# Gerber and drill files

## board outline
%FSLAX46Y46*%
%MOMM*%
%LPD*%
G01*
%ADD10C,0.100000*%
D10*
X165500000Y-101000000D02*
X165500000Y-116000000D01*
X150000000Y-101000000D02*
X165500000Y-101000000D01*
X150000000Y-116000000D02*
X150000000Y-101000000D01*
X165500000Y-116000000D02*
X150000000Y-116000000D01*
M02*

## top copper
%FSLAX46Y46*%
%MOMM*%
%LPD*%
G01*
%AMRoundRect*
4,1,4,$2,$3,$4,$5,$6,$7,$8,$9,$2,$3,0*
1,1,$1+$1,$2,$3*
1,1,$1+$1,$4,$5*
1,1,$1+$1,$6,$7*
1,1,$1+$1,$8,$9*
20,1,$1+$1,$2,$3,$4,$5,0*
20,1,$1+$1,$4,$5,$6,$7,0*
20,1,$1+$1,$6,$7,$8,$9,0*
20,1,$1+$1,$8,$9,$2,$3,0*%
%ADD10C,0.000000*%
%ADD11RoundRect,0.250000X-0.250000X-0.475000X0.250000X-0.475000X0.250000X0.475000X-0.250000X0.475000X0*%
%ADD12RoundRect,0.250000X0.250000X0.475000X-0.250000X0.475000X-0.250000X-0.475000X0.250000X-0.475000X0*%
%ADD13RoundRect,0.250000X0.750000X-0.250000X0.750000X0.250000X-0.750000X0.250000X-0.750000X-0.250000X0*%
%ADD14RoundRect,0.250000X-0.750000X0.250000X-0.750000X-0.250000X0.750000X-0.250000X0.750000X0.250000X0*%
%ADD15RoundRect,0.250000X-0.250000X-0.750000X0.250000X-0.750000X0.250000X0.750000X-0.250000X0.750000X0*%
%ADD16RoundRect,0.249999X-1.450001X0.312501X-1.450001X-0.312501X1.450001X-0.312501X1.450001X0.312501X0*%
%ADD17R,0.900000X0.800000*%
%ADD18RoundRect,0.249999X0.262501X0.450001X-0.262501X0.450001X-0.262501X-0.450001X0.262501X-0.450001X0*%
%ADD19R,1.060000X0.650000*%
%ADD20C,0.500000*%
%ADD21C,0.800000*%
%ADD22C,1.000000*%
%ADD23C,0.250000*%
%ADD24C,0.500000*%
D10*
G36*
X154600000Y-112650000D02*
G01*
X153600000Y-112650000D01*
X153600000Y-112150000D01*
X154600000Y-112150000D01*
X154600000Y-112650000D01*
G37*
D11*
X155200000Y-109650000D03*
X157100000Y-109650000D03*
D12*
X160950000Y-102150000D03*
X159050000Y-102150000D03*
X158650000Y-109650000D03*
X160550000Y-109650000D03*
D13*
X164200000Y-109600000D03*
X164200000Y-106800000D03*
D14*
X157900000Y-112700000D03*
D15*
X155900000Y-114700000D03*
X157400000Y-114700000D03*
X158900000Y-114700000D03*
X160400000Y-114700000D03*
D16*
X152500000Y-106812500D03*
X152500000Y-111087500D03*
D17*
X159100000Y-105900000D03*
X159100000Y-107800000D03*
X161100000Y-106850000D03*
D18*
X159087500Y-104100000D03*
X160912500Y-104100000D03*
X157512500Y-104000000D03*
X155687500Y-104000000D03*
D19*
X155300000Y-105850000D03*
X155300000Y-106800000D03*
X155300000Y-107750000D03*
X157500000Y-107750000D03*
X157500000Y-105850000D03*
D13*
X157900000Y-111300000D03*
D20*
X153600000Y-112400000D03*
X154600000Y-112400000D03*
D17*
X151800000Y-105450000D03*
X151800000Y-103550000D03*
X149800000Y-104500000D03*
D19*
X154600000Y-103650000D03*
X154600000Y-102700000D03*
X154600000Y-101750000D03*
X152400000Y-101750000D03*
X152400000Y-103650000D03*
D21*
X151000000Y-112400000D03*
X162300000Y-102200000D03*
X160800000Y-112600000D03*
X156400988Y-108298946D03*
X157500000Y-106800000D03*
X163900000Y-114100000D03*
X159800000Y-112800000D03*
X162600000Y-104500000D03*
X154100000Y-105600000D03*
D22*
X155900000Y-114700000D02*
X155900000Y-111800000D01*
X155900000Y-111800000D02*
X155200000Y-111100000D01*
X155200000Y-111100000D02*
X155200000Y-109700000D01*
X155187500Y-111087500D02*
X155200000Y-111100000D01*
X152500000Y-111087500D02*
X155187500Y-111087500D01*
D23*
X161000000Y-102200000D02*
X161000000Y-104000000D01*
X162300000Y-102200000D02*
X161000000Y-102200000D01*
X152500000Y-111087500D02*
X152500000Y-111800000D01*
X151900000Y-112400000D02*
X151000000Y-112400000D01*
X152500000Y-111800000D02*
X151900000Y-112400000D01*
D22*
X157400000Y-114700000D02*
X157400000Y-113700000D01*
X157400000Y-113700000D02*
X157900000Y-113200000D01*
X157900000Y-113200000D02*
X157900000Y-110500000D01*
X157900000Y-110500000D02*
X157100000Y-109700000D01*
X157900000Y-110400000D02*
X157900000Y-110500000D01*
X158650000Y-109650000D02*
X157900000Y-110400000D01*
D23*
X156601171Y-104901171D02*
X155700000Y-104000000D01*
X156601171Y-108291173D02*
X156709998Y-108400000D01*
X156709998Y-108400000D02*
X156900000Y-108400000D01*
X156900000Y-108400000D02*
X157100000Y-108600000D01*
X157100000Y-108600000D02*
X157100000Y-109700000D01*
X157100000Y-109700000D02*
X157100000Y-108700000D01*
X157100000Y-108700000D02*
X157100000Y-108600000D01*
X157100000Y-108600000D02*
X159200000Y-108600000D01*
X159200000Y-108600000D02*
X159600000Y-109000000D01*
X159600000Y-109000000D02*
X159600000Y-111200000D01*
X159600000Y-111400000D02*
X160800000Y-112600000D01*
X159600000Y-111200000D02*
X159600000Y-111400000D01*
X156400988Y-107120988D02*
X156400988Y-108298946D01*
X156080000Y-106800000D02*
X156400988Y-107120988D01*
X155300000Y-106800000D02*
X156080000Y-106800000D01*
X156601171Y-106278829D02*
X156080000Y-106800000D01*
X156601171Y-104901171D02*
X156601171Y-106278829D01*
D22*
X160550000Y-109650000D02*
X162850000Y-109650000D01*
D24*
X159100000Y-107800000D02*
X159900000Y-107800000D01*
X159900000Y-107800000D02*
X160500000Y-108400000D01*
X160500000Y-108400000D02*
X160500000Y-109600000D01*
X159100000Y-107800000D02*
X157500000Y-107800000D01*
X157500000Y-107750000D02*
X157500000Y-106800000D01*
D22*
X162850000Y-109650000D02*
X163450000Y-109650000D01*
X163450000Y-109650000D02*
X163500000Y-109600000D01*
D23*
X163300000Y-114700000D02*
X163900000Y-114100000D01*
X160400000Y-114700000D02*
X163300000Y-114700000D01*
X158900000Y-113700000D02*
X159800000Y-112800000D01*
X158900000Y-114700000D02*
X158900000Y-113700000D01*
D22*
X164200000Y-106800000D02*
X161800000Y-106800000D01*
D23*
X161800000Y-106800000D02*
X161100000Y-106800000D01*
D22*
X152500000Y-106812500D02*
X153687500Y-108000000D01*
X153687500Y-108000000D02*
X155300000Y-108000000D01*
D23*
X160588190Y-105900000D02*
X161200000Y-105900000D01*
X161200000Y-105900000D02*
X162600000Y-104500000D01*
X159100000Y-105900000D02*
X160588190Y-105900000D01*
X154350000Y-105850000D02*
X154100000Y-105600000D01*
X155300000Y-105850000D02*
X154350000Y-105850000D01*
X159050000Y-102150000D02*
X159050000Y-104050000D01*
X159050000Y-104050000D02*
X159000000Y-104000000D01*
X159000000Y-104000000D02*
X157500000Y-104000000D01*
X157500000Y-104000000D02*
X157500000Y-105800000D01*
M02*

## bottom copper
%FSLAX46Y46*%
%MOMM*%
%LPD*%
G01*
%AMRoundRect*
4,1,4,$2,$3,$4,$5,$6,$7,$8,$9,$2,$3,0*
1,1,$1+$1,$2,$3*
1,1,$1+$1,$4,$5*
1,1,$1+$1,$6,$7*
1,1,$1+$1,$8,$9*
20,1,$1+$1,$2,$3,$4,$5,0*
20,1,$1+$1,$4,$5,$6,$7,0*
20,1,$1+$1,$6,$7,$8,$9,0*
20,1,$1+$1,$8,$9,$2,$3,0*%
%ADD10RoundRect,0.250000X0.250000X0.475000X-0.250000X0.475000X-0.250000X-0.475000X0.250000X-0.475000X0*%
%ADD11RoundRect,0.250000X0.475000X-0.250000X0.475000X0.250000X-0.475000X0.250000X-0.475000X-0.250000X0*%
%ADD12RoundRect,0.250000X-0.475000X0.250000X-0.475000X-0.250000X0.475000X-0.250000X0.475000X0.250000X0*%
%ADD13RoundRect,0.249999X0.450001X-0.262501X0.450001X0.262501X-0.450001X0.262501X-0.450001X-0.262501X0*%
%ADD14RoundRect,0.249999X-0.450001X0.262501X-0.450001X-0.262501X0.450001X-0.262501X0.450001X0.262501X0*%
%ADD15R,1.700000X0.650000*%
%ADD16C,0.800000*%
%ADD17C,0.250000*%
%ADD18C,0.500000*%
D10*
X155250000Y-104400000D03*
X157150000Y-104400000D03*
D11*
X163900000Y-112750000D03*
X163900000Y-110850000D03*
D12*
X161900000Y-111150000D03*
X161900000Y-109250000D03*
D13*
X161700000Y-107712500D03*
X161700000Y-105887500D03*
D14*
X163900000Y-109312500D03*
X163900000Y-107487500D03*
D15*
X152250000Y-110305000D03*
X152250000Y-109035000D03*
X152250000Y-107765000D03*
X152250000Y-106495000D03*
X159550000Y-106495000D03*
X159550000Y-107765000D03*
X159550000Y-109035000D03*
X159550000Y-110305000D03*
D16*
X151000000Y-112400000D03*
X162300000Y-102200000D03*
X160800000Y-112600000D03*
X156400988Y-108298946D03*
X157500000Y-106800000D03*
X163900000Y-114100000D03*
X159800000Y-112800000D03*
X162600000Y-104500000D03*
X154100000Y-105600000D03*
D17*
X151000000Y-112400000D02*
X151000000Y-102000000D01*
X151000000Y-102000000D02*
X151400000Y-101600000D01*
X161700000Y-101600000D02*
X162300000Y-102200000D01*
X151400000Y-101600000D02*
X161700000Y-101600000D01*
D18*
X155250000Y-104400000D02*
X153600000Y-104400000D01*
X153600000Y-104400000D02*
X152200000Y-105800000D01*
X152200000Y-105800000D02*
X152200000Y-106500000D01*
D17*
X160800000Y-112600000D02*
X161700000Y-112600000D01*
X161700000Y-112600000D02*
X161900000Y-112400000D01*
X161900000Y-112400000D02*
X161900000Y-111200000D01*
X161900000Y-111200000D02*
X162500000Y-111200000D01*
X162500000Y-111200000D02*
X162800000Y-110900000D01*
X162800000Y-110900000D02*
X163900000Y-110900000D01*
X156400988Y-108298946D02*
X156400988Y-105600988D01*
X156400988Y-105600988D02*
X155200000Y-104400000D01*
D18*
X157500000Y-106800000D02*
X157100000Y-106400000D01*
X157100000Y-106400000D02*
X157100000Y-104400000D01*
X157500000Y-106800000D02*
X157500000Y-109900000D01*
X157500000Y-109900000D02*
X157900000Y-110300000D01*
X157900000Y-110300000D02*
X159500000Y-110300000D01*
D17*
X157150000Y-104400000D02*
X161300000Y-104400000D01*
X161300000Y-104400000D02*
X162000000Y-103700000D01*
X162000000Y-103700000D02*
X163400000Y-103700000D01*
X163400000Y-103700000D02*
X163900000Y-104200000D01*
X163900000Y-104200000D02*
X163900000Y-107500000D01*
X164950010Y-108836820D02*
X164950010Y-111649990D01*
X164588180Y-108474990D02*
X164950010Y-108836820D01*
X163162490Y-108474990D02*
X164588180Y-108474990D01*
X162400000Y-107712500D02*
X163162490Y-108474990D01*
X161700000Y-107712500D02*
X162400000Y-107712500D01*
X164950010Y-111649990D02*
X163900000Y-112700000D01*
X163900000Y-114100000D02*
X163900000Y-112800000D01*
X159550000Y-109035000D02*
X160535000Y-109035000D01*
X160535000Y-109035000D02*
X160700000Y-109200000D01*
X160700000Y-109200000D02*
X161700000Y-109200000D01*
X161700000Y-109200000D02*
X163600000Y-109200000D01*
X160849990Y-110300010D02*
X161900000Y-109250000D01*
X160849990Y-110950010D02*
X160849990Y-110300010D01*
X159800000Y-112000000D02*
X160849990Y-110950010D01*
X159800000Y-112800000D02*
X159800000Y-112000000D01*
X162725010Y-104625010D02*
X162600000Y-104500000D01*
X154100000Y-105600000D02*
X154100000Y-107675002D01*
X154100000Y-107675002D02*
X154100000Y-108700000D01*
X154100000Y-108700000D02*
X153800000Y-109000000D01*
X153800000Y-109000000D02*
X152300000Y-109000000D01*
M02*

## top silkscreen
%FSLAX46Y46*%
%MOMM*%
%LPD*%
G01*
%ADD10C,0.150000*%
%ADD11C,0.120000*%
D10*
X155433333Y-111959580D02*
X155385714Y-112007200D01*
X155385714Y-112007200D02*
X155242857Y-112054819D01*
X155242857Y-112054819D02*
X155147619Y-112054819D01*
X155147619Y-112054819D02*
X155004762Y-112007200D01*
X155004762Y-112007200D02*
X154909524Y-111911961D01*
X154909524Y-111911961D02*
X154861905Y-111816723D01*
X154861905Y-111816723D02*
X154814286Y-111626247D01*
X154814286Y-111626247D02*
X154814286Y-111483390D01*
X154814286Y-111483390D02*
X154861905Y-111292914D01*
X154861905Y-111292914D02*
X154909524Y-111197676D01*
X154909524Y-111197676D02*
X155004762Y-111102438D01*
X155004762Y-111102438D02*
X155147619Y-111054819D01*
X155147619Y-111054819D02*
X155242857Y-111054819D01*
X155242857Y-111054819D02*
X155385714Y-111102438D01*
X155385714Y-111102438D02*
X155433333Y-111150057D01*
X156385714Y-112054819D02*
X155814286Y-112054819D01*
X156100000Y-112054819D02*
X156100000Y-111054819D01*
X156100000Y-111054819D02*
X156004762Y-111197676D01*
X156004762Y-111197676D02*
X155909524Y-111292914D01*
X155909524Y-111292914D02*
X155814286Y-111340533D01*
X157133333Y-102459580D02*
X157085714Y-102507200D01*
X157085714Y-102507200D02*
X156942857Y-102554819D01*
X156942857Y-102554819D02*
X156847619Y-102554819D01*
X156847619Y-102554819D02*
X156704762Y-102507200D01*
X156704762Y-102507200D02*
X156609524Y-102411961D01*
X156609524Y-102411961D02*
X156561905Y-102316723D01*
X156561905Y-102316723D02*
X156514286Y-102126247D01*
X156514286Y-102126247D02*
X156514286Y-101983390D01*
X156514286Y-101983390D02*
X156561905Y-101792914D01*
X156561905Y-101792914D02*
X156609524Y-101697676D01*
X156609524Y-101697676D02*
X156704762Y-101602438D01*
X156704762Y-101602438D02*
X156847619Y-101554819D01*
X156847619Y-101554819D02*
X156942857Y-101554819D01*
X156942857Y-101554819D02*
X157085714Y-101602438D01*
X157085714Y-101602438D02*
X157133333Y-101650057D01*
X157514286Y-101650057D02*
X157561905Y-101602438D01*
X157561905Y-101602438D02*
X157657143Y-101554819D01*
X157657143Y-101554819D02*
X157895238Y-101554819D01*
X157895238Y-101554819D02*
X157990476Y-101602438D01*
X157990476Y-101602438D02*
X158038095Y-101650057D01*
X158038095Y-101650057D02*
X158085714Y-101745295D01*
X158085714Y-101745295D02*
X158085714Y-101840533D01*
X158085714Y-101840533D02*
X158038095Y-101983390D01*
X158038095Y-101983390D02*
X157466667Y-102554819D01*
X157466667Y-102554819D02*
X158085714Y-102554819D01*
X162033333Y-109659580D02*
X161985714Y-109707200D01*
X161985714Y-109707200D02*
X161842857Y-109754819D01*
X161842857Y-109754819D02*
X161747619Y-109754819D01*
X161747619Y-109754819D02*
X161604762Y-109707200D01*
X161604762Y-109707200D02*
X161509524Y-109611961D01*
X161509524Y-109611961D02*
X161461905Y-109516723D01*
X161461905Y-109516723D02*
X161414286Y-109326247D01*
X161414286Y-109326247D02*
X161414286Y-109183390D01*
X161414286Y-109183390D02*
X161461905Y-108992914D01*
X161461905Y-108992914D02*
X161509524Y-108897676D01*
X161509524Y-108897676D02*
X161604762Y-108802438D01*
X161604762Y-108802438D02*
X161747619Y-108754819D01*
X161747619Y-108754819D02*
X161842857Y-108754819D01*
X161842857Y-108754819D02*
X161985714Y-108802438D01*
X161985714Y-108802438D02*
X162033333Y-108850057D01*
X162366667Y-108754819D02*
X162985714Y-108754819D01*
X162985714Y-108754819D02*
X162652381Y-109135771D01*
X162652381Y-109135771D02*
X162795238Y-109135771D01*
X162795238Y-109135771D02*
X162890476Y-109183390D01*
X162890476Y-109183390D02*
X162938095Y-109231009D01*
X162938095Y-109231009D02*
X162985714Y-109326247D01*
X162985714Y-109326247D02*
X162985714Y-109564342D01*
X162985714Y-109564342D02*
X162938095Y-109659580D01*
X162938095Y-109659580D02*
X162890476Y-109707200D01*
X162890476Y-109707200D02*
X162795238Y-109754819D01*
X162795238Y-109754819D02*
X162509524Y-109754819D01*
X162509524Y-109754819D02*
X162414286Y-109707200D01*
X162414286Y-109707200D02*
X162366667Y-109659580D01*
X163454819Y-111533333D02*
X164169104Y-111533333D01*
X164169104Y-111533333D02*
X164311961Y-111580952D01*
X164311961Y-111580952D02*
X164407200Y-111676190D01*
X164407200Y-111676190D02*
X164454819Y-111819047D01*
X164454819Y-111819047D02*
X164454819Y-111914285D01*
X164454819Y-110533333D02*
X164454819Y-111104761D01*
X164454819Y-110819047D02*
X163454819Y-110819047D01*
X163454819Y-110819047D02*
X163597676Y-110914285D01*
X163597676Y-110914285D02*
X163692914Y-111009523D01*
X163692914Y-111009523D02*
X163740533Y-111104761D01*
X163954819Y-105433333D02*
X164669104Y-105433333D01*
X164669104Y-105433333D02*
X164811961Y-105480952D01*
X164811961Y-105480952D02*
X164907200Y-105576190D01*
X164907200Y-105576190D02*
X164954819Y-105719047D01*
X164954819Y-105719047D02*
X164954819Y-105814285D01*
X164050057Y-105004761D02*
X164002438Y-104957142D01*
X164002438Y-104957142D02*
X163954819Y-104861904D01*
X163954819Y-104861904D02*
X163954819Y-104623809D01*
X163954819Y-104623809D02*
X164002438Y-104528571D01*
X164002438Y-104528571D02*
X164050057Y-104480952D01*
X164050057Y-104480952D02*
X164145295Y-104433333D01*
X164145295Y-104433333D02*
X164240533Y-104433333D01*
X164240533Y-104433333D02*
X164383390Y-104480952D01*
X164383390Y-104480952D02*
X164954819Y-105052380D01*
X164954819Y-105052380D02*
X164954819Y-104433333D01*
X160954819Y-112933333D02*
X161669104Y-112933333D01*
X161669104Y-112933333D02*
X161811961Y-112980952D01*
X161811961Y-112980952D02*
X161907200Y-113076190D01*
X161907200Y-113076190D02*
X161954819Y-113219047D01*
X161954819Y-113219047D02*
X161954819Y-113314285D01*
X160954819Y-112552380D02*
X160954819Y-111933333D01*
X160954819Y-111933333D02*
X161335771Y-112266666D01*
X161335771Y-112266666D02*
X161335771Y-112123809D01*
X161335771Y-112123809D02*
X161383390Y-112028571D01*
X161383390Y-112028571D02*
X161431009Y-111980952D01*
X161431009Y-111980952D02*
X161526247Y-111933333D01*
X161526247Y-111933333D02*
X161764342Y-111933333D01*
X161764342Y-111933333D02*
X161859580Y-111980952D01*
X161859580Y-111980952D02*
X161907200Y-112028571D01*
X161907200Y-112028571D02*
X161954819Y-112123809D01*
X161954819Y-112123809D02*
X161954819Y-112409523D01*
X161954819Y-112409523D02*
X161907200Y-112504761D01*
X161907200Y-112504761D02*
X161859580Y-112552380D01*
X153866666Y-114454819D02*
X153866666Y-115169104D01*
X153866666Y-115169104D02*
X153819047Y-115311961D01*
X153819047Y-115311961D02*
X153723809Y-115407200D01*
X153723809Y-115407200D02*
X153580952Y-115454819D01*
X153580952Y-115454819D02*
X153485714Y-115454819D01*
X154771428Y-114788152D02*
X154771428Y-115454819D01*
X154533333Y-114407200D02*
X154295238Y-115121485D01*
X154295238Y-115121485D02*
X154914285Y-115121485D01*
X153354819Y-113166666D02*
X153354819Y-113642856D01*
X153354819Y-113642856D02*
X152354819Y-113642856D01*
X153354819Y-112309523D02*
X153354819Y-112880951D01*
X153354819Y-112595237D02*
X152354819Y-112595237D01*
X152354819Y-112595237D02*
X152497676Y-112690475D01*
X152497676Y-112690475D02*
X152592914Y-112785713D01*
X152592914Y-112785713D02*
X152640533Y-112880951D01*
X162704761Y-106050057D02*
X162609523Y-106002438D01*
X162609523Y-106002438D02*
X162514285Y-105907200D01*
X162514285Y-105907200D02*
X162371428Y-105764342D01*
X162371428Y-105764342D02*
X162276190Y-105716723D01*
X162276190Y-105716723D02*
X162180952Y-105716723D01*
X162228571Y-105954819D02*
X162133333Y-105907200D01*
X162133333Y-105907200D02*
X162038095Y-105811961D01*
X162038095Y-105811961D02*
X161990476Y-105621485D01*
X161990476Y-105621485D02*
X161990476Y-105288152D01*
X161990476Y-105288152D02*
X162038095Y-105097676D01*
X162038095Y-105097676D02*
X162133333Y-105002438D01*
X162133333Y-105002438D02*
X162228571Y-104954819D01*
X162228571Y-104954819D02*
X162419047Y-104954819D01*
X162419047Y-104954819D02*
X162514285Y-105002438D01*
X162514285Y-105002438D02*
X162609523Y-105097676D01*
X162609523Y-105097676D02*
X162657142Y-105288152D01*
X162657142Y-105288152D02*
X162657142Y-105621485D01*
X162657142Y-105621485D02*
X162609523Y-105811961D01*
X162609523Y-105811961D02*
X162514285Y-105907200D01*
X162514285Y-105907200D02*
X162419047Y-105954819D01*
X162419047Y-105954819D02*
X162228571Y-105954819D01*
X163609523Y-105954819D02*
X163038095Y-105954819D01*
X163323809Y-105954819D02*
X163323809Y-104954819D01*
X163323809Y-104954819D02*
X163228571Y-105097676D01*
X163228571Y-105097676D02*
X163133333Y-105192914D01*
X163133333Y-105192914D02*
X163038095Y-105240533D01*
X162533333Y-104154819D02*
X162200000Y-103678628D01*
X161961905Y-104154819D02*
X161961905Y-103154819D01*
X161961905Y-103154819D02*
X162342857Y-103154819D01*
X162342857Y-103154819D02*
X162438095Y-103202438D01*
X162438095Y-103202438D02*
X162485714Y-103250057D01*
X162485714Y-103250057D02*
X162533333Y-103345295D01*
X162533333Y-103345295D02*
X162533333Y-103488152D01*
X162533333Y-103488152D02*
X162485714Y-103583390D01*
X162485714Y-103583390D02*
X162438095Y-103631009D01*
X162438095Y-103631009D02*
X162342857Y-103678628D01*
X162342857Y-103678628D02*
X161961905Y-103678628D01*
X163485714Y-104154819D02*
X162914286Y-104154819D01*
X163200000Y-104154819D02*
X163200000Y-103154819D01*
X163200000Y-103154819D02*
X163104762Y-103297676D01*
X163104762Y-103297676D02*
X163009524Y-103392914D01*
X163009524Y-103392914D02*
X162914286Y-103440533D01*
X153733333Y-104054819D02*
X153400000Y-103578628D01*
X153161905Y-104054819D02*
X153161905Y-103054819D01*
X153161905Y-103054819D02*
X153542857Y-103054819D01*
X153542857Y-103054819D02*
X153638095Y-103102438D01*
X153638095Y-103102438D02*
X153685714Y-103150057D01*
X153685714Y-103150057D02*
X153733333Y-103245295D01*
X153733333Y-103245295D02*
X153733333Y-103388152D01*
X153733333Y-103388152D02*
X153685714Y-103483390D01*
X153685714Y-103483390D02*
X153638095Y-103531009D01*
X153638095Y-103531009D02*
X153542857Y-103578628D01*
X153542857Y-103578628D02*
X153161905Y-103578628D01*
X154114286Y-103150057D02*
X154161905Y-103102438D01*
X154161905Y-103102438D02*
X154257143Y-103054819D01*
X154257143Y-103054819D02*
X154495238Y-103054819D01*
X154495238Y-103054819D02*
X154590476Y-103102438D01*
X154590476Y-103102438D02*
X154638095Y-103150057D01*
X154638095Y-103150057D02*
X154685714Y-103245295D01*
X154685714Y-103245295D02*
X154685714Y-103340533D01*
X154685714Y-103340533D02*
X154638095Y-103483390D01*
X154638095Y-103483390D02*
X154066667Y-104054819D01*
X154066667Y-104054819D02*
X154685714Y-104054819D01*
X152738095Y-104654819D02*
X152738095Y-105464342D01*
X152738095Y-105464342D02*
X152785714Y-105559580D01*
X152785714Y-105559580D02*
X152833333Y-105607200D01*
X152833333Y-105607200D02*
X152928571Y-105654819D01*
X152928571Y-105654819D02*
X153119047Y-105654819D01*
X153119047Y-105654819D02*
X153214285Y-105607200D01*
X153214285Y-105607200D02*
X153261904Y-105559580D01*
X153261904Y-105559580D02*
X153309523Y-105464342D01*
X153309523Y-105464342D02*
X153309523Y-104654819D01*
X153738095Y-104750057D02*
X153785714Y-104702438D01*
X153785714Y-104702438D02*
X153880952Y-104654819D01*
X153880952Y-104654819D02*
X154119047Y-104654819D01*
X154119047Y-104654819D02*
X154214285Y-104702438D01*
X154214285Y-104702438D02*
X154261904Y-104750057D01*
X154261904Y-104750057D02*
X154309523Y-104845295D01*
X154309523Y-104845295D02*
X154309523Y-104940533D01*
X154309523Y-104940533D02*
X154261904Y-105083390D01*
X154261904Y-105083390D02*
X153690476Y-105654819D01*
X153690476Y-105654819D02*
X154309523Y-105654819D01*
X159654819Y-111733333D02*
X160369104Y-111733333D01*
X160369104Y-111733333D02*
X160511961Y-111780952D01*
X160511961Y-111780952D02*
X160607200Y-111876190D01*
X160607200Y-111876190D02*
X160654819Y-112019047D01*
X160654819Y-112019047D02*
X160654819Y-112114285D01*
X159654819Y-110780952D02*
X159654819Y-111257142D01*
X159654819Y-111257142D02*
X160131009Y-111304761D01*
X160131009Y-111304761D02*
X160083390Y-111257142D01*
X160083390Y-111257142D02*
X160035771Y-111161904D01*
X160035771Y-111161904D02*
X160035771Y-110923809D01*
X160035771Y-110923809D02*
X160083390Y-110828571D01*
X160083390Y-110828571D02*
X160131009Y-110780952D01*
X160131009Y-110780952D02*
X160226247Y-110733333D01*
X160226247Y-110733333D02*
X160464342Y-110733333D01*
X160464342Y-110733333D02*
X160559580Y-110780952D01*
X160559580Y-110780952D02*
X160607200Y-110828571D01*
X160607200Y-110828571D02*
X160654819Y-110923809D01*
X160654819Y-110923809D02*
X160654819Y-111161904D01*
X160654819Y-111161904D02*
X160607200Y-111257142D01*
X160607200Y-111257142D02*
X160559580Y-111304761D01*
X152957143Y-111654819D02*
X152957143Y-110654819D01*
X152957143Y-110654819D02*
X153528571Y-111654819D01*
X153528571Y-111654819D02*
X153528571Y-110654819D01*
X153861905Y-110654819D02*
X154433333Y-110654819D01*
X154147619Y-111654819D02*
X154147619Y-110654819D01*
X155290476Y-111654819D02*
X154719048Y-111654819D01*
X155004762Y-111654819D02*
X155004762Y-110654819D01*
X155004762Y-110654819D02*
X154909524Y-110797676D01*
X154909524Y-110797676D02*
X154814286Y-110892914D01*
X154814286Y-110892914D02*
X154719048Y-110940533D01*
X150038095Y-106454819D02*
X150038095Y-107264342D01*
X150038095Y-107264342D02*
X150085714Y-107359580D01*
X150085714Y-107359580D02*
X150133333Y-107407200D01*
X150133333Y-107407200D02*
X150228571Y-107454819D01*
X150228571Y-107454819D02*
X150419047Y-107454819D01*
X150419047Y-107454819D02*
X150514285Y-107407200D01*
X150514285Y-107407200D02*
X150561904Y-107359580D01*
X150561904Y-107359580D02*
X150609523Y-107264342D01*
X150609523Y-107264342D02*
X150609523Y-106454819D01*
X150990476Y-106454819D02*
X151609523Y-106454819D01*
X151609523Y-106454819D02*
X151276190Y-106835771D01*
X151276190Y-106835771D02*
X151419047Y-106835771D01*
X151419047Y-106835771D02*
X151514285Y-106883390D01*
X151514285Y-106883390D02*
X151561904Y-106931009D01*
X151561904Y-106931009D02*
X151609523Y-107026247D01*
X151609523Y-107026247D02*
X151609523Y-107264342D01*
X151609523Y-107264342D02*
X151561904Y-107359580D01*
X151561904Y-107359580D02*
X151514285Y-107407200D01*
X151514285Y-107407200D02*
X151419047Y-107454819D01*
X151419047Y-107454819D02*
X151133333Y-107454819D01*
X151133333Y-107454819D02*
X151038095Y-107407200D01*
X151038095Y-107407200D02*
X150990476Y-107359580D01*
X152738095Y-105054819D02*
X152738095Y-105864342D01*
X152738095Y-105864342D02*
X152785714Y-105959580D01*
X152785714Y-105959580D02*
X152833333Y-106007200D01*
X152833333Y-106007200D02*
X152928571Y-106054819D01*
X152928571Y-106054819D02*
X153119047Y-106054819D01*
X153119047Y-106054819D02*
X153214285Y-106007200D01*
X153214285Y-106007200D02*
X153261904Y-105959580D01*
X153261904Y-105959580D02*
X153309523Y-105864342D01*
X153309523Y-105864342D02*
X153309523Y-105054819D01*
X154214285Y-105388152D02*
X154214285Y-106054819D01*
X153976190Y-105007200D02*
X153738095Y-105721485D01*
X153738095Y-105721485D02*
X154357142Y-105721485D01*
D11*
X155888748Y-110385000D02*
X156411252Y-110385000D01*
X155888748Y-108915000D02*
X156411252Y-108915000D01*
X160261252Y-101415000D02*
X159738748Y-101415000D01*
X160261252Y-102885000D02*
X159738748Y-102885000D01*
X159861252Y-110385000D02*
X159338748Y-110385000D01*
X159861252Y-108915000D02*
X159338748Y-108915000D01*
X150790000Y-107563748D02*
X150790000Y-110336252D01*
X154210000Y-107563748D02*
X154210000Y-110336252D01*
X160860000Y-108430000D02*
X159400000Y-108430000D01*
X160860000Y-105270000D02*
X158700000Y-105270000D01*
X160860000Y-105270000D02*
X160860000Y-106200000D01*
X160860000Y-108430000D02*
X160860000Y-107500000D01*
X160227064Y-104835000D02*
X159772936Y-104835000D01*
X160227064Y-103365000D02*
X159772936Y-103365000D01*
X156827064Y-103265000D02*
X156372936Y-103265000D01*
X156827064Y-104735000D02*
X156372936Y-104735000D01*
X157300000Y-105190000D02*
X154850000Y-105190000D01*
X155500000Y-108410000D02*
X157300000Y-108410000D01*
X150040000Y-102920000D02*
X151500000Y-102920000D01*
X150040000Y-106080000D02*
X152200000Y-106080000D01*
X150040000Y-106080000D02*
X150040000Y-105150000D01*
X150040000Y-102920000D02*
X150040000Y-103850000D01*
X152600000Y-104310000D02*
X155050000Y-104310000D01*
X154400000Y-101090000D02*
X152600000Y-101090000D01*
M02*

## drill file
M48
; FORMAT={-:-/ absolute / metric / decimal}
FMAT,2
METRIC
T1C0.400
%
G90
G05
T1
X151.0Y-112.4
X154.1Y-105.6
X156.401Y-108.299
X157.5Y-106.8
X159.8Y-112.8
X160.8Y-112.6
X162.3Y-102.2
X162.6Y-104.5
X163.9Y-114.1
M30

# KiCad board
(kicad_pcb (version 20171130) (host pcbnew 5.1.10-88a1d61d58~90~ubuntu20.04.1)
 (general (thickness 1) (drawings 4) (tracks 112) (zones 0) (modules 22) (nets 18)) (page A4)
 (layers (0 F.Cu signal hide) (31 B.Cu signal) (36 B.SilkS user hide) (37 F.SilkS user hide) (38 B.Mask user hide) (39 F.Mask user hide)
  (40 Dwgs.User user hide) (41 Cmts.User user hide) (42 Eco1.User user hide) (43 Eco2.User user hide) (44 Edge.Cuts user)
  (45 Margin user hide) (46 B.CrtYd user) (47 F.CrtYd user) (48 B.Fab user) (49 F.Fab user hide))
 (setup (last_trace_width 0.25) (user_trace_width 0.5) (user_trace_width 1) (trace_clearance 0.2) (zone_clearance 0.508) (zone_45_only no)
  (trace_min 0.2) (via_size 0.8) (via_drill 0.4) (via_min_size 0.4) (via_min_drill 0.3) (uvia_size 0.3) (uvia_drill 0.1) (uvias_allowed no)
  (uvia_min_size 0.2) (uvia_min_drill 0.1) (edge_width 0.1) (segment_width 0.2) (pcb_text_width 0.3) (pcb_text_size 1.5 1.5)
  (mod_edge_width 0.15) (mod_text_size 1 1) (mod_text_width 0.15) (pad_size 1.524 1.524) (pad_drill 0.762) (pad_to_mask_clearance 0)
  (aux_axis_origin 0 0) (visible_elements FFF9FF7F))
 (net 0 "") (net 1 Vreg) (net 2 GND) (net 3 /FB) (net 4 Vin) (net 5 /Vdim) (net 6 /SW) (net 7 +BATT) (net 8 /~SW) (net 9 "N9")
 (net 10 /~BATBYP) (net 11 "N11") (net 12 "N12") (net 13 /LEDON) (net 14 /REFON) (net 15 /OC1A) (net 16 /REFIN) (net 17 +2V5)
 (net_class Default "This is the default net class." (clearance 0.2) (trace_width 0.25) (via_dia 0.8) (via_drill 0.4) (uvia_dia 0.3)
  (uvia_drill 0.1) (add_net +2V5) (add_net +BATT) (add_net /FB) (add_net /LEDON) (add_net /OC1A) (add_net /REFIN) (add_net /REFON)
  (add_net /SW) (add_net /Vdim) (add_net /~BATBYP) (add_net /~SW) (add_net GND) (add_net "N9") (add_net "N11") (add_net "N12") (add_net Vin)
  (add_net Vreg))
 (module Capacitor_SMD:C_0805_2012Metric (layer F.Cu) (at 156.15 109.65)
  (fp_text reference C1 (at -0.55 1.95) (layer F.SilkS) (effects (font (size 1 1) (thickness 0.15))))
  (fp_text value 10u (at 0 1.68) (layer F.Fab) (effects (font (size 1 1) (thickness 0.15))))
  (fp_line (start -0.261252 0.735) (end 0.261252 0.735) (layer F.SilkS) (width 0.12))
  (fp_line (start -0.261252 -0.735) (end 0.261252 -0.735) (layer F.SilkS) (width 0.12))
  (pad 1 smd roundrect (at -0.95 0) (size 1 1.45) (layers F.Cu F.Paste F.Mask) (roundrect_rratio 0.25) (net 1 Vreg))
  (pad 2 smd roundrect (at 0.95 0) (size 1 1.45) (layers F.Cu F.Paste F.Mask) (roundrect_rratio 0.25) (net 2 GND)))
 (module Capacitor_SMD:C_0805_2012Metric (layer F.Cu) (at 160 102.15 180)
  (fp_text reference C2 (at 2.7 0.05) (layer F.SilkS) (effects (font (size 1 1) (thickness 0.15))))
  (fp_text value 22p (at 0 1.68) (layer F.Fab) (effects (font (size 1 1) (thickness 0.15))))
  (fp_line (start -0.261252 0.735) (end 0.261252 0.735) (layer F.SilkS) (width 0.12))
  (fp_line (start -0.261252 -0.735) (end 0.261252 -0.735) (layer F.SilkS) (width 0.12))
  (pad 1 smd roundrect (at -0.95 0 180) (size 1 1.45) (layers F.Cu F.Paste F.Mask) (roundrect_rratio 0.25) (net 1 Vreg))
  (pad 2 smd roundrect (at 0.95 0 180) (size 1 1.45) (layers F.Cu F.Paste F.Mask) (roundrect_rratio 0.25) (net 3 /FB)))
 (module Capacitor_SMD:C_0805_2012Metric (layer F.Cu) (at 159.6 109.65 180)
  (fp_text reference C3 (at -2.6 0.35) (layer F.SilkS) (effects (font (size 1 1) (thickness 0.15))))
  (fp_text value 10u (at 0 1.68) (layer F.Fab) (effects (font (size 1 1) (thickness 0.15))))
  (fp_line (start -0.261252 -0.735) (end 0.261252 -0.735) (layer F.SilkS) (width 0.12))
  (fp_line (start -0.261252 0.735) (end 0.261252 0.735) (layer F.SilkS) (width 0.12))
  (pad 2 smd roundrect (at 0.95 0 180) (size 1 1.45) (layers F.Cu F.Paste F.Mask) (roundrect_rratio 0.25) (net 2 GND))
  (pad 1 smd roundrect (at -0.95 0 180) (size 1 1.45) (layers F.Cu F.Paste F.Mask) (roundrect_rratio 0.25) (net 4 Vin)))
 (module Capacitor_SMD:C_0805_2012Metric (layer B.Cu) (at 156.2 104.4 180)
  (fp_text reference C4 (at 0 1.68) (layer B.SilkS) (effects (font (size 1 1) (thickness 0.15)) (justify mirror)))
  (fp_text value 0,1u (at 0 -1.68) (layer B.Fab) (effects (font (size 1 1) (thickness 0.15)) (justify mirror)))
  (pad 2 smd roundrect (at 0.95 0 180) (size 1 1.45) (layers B.Cu B.Paste B.Mask) (roundrect_rratio 0.25) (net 2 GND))
  (pad 1 smd roundrect (at -0.95 0 180) (size 1 1.45) (layers B.Cu B.Paste B.Mask) (roundrect_rratio 0.25) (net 4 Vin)))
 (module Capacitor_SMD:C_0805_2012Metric (layer B.Cu) (at 163.9 111.8 90)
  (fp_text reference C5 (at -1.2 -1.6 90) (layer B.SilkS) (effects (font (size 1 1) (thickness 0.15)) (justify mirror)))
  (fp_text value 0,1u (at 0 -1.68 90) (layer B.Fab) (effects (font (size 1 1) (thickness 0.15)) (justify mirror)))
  (pad 1 smd roundrect (at -0.95 0 90) (size 1 1.45) (layers B.Cu B.Paste B.Mask) (roundrect_rratio 0.25) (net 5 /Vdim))
  (pad 2 smd roundrect (at 0.95 0 90) (size 1 1.45) (layers B.Cu B.Paste B.Mask) (roundrect_rratio 0.25) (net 2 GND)))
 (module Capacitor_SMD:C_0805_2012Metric (layer B.Cu) (at 161.9 110.2 270)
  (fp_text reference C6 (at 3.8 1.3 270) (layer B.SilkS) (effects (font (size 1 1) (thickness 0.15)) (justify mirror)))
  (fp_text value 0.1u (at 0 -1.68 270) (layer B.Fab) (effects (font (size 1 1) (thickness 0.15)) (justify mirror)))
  (pad 2 smd roundrect (at 0.95 0 270) (size 1 1.45) (layers B.Cu B.Paste B.Mask) (roundrect_rratio 0.25) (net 2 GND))
  (pad 1 smd roundrect (at -0.95 0 270) (size 1 1.45) (layers B.Cu B.Paste B.Mask) (roundrect_rratio 0.25) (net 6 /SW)))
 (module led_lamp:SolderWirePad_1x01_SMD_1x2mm (layer F.Cu) (at 164.2 109.6 90)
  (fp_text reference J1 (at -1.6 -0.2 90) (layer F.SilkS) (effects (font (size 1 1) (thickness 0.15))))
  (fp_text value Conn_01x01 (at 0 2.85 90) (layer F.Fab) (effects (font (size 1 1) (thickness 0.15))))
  (pad 1 smd roundrect (at 0 0 90) (size 1 2) (layers F.Cu F.Paste F.Mask) (roundrect_rratio 0.25) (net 4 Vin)))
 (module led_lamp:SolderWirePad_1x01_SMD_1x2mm (layer F.Cu) (at 164.2 106.8 90)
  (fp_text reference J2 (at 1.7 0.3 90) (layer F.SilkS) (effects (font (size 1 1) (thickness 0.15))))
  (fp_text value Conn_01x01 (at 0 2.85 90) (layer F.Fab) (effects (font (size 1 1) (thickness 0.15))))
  (pad 1 smd roundrect (at 0 0 90) (size 1 2) (layers F.Cu F.Paste F.Mask) (roundrect_rratio 0.25) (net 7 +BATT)))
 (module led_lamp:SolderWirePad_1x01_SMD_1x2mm (layer F.Cu) (at 157.9 112.7 270)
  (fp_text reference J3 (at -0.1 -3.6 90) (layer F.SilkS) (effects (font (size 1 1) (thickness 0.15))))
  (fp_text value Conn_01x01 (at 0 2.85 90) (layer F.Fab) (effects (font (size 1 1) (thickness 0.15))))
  (pad 1 smd roundrect (at 0 0 270) (size 1 2) (layers F.Cu F.Paste F.Mask) (roundrect_rratio 0.25) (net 2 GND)))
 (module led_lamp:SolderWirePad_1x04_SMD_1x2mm (layer F.Cu) (at 155.9 114.7)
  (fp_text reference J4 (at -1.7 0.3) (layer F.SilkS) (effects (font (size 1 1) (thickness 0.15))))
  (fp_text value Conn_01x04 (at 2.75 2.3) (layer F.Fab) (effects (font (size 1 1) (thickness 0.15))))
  (pad 1 smd roundrect (at 0 0) (size 1 2) (layers F.Cu F.Paste F.Mask) (roundrect_rratio 0.25) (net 1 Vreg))
  (pad 2 smd roundrect (at 1.5 0) (size 1 2) (layers F.Cu F.Paste F.Mask) (roundrect_rratio 0.25) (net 2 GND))
  (pad 3 smd roundrect (at 3 0) (size 1 2) (layers F.Cu F.Paste F.Mask) (roundrect_rratio 0.25) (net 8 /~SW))
  (pad 4 smd roundrect (at 4.5 0) (size 1 2) (layers F.Cu F.Paste F.Mask) (roundrect_rratio 0.25) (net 5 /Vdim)))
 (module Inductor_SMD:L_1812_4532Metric (layer F.Cu) (at 152.5 108.95 270)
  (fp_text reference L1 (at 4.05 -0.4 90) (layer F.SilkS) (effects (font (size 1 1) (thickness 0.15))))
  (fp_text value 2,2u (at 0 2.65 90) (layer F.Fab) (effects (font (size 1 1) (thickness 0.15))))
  (fp_line (start -1.386252 1.71) (end 1.386252 1.71) (layer F.SilkS) (width 0.12))
  (fp_line (start -1.386252 -1.71) (end 1.386252 -1.71) (layer F.SilkS) (width 0.12))
  (pad 1 smd roundrect (at -2.1375 0 270) (size 1.125 3.4) (layers F.Cu F.Paste F.Mask) (roundrect_rratio 0.2222213333333333) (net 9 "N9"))
  (pad 2 smd roundrect (at 2.1375 0 270) (size 1.125 3.4) (layers F.Cu F.Paste F.Mask) (roundrect_rratio 0.2222213333333333) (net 1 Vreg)))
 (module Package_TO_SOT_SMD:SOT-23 (layer F.Cu) (at 160.1 106.85)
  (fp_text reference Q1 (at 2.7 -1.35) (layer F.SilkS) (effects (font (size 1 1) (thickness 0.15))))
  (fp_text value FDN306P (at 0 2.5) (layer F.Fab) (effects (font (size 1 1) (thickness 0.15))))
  (fp_line (start 0.76 1.58) (end -0.7 1.58) (layer F.SilkS) (width 0.12))
  (fp_line (start 0.76 -1.58) (end -1.4 -1.58) (layer F.SilkS) (width 0.12))
  (fp_line (start 0.76 -1.58) (end 0.76 -0.65) (layer F.SilkS) (width 0.12))
  (fp_line (start 0.76 1.58) (end 0.76 0.65) (layer F.SilkS) (width 0.12))
  (pad 1 smd rect (at -1 -0.95) (size 0.9 0.8) (layers F.Cu F.Paste F.Mask) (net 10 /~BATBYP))
  (pad 2 smd rect (at -1 0.95) (size 0.9 0.8) (layers F.Cu F.Paste F.Mask) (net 4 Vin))
  (pad 3 smd rect (at 1 0) (size 0.9 0.8) (layers F.Cu F.Paste F.Mask) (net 7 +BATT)))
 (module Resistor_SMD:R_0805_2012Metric (layer F.Cu) (at 160 104.1 180)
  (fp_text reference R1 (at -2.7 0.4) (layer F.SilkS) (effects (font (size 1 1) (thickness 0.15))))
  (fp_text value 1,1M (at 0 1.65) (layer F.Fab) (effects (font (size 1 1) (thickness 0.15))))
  (fp_line (start -0.227064 -0.735) (end 0.227064 -0.735) (layer F.SilkS) (width 0.12))
  (fp_line (start -0.227064 0.735) (end 0.227064 0.735) (layer F.SilkS) (width 0.12))
  (pad 2 smd roundrect (at 0.9125 0 180) (size 1.025 1.4) (layers F.Cu F.Paste F.Mask) (roundrect_rratio 0.2439014634146341) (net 3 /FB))
  (pad 1 smd roundrect (at -0.9125 0 180) (size 1.025 1.4) (layers F.Cu F.Paste F.Mask) (roundrect_rratio 0.2439014634146341) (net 1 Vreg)))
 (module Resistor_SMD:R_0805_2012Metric (layer F.Cu) (at 156.6 104 180)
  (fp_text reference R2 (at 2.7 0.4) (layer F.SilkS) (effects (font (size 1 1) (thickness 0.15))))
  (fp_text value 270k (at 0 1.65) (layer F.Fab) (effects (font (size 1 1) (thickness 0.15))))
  (fp_line (start -0.227064 0.735) (end 0.227064 0.735) (layer F.SilkS) (width 0.12))
  (fp_line (start -0.227064 -0.735) (end 0.227064 -0.735) (layer F.SilkS) (width 0.12))
  (pad 1 smd roundrect (at -0.9125 0 180) (size 1.025 1.4) (layers F.Cu F.Paste F.Mask) (roundrect_rratio 0.2439014634146341) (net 3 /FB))
  (pad 2 smd roundrect (at 0.9125 0 180) (size 1.025 1.4) (layers F.Cu F.Paste F.Mask) (roundrect_rratio 0.2439014634146341) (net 2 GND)))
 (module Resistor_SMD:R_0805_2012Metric (layer B.Cu) (at 161.7 106.8 90)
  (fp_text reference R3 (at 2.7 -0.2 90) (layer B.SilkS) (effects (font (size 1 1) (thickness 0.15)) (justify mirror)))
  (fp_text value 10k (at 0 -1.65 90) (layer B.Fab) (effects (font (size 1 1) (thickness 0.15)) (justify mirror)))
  (pad 1 smd roundrect (at -0.9125 0 90) (size 1.025 1.4) (layers B.Cu B.Paste B.Mask) (roundrect_rratio 0.2439014634146341) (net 5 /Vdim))
  (pad 2 smd roundrect (at 0.9125 0 90) (size 1.025 1.4) (layers B.Cu B.Paste B.Mask) (roundrect_rratio 0.2439014634146341) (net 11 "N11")))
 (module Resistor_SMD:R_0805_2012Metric (layer B.Cu) (at 163.9 108.4 270)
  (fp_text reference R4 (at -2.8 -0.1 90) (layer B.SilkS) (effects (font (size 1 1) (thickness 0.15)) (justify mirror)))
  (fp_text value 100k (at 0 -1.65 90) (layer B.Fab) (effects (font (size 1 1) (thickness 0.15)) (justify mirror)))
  (pad 2 smd roundrect (at 0.9125 0 270) (size 1.025 1.4) (layers B.Cu B.Paste B.Mask) (roundrect_rratio 0.2439014634146341) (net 8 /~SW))
  (pad 1 smd roundrect (at -0.9125 0 270) (size 1.025 1.4) (layers B.Cu B.Paste B.Mask) (roundrect_rratio 0.2439014634146341) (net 4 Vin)))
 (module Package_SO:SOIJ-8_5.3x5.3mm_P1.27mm (layer B.Cu) (at 155.9 108.4)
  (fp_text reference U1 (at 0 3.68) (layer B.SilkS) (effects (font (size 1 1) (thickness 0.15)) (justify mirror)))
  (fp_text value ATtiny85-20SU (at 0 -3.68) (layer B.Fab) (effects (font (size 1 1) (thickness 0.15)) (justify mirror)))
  (pad 1 smd rect (at -3.65 1.905) (size 1.7 0.65) (layers B.Cu B.Paste B.Mask) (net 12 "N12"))
  (pad 2 smd rect (at -3.65 0.635) (size 1.7 0.65) (layers B.Cu B.Paste B.Mask) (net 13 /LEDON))
  (pad 3 smd rect (at -3.65 -0.635) (size 1.7 0.65) (layers B.Cu B.Paste B.Mask) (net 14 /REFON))
  (pad 4 smd rect (at -3.65 -1.905) (size 1.7 0.65) (layers B.Cu B.Paste B.Mask) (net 2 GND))
  (pad 5 smd rect (at 3.65 -1.905) (size 1.7 0.65) (layers B.Cu B.Paste B.Mask) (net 10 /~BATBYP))
  (pad 6 smd rect (at 3.65 -0.635) (size 1.7 0.65) (layers B.Cu B.Paste B.Mask) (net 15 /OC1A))
  (pad 7 smd rect (at 3.65 0.635) (size 1.7 0.65) (layers B.Cu B.Paste B.Mask) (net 8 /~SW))
  (pad 8 smd rect (at 3.65 1.905) (size 1.7 0.65) (layers B.Cu B.Paste B.Mask) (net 4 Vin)))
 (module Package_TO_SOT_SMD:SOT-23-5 (layer F.Cu) (at 156.4 106.8)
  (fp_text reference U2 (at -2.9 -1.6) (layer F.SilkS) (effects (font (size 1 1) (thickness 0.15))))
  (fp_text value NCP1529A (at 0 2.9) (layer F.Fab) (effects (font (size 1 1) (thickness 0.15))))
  (fp_line (start 0.9 -1.61) (end -1.55 -1.61) (layer F.SilkS) (width 0.12))
  (fp_line (start -0.9 1.61) (end 0.9 1.61) (layer F.SilkS) (width 0.12))
  (pad 1 smd rect (at -1.1 -0.95) (size 1.06 0.65) (layers F.Cu F.Paste F.Mask) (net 13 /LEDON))
  (pad 2 smd rect (at -1.1 0) (size 1.06 0.65) (layers F.Cu F.Paste F.Mask) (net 2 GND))
  (pad 3 smd rect (at -1.1 0.95) (size 1.06 0.65) (layers F.Cu F.Paste F.Mask) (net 9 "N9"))
  (pad 4 smd rect (at 1.1 0.95) (size 1.06 0.65) (layers F.Cu F.Paste F.Mask) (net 4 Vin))
  (pad 5 smd rect (at 1.1 -0.95) (size 1.06 0.65) (layers F.Cu F.Paste F.Mask) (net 3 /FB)))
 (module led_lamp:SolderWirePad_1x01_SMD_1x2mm (layer F.Cu) (at 157.9 111.3 90)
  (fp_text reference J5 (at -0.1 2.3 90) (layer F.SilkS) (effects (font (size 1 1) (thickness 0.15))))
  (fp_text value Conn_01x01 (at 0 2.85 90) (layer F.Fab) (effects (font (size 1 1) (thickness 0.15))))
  (pad 1 smd roundrect (at 0 0 90) (size 1 2) (layers F.Cu F.Paste F.Mask) (roundrect_rratio 0.25) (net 2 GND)))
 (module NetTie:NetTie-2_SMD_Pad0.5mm (layer F.Cu) (at 154.1 112.4)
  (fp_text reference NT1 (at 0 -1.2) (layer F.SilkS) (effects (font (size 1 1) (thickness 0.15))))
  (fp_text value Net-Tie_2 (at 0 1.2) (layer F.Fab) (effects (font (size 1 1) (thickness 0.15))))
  (fp_poly (pts (xy -0.5 -0.25) (xy 0.5 -0.25) (xy 0.5 0.25) (xy -0.5 0.25)) (layer F.Cu) (width 0))
  (pad 1 smd circle (at -0.5 0) (size 0.5 0.5) (layers F.Cu) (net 14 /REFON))
  (pad 2 smd circle (at 0.5 0) (size 0.5 0.5) (layers F.Cu) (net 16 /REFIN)))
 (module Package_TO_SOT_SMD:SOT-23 (layer F.Cu) (at 150.8 104.5 180)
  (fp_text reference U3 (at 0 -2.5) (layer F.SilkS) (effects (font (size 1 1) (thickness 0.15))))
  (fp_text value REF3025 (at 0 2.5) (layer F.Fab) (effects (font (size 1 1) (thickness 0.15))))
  (fp_line (start 0.76 1.58) (end -0.7 1.58) (layer F.SilkS) (width 0.12))
  (fp_line (start 0.76 -1.58) (end -1.4 -1.58) (layer F.SilkS) (width 0.12))
  (fp_line (start 0.76 -1.58) (end 0.76 -0.65) (layer F.SilkS) (width 0.12))
  (fp_line (start 0.76 1.58) (end 0.76 0.65) (layer F.SilkS) (width 0.12))
  (pad 1 smd rect (at -1 -0.95 180) (size 0.9 0.8) (layers F.Cu F.Paste F.Mask) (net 16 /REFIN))
  (pad 2 smd rect (at -1 0.95 180) (size 0.9 0.8) (layers F.Cu F.Paste F.Mask) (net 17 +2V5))
  (pad 3 smd rect (at 1 0 180) (size 0.9 0.8) (layers F.Cu F.Paste F.Mask) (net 2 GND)))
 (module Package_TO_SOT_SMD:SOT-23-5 (layer F.Cu) (at 153.5 102.7 180)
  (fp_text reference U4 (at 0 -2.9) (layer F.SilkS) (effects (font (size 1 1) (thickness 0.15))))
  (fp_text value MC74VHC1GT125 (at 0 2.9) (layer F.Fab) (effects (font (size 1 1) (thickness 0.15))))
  (fp_line (start 0.9 -1.61) (end -1.55 -1.61) (layer F.SilkS) (width 0.12))
  (fp_line (start -0.9 1.61) (end 0.9 1.61) (layer F.SilkS) (width 0.12))
  (pad 1 smd rect (at -1.1 -0.95 180) (size 1.06 0.65) (layers F.Cu F.Paste F.Mask) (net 2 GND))
  (pad 2 smd rect (at -1.1 0 180) (size 1.06 0.65) (layers F.Cu F.Paste F.Mask) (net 15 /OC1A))
  (pad 3 smd rect (at -1.1 0.95 180) (size 1.06 0.65) (layers F.Cu F.Paste F.Mask) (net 2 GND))
  (pad 4 smd rect (at 1.1 0.95 180) (size 1.06 0.65) (layers F.Cu F.Paste F.Mask) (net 11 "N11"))
  (pad 5 smd rect (at 1.1 -0.95 180) (size 1.06 0.65) (layers F.Cu F.Paste F.Mask) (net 17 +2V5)))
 (gr_line (start 165.5 101) (end 165.5 116) (layer Edge.Cuts) (width 0.1))
 (gr_line (start 150 101) (end 165.5 101) (layer Edge.Cuts) (width 0.1))
 (gr_line (start 150 116) (end 150 101) (layer Edge.Cuts) (width 0.1))
 (gr_line (start 165.5 116) (end 150 116) (layer Edge.Cuts) (width 0.1))
 (segment (start 155.9 114.7) (end 155.9 111.8) (width 1) (layer F.Cu) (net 1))
 (segment (start 155.9 111.8) (end 155.2 111.1) (width 1) (layer F.Cu) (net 1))
 (segment (start 155.2 111.1) (end 155.2 109.7) (width 1) (layer F.Cu) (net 1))
 (segment (start 155.1875 111.0875) (end 155.2 111.1) (width 1) (layer F.Cu) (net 1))
 (segment (start 152.5 111.0875) (end 155.1875 111.0875) (width 1) (layer F.Cu) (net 1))
 (segment (start 161 102.2) (end 161 104) (width 0.25) (layer F.Cu) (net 1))
 (via (at 151 112.4) (size 0.8) (drill 0.4) (layers F.Cu B.Cu) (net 1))
 (segment (start 162.3 102.2) (end 161 102.2) (width 0.25) (layer F.Cu) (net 1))
 (via (at 162.3 102.2) (size 0.8) (drill 0.4) (layers F.Cu B.Cu) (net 1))
 (segment (start 152.5 111.0875) (end 152.5 111.8) (width 0.25) (layer F.Cu) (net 1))
 (segment (start 151.9 112.4) (end 151 112.4) (width 0.25) (layer F.Cu) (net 1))
 (segment (start 152.5 111.8) (end 151.9 112.4) (width 0.25) (layer F.Cu) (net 1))
 (segment (start 151 112.4) (end 151 102) (width 0.25) (layer B.Cu) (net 1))
 (segment (start 151 102) (end 151.4 101.6) (width 0.25) (layer B.Cu) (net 1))
 (segment (start 161.7 101.6) (end 162.3 102.2) (width 0.25) (layer B.Cu) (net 1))
 (segment (start 151.4 101.6) (end 161.7 101.6) (width 0.25) (layer B.Cu) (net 1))
 (segment (start 157.4 114.7) (end 157.4 113.7) (width 1) (layer F.Cu) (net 2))
 (segment (start 157.4 113.7) (end 157.9 113.2) (width 1) (layer F.Cu) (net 2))
 (segment (start 157.9 113.2) (end 157.9 110.5) (width 1) (layer F.Cu) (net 2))
 (segment (start 157.9 110.5) (end 157.1 109.7) (width 1) (layer F.Cu) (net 2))
 (segment (start 157.9 110.4) (end 157.9 110.5) (width 1) (layer F.Cu) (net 2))
 (segment (start 158.65 109.65) (end 157.9 110.4) (width 1) (layer F.Cu) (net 2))
 (segment (start 156.601171 104.901171) (end 155.7 104) (width 0.25) (layer F.Cu) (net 2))
 (segment (start 155.25 104.4) (end 153.6 104.4) (width 0.5) (layer B.Cu) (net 2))
 (segment (start 153.6 104.4) (end 152.2 105.8) (width 0.5) (layer B.Cu) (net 2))
 (segment (start 152.2 105.8) (end 152.2 106.5) (width 0.5) (layer B.Cu) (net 2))
 (segment (start 156.601171 108.291173) (end 156.709998 108.4) (width 0.25) (layer F.Cu) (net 2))
 (segment (start 156.709998 108.4) (end 156.9 108.4) (width 0.25) (layer F.Cu) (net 2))
 (segment (start 156.9 108.4) (end 157.1 108.6) (width 0.25) (layer F.Cu) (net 2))
 (segment (start 157.1 108.6) (end 157.1 109.7) (width 0.25) (layer F.Cu) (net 2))
 (segment (start 157.1 109.7) (end 157.1 108.7) (width 0.25) (layer F.Cu) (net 2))
 (segment (start 157.1 108.7) (end 157.1 108.6) (width 0.25) (layer F.Cu) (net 2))
 (segment (start 157.1 108.6) (end 159.2 108.6) (width 0.25) (layer F.Cu) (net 2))
 (segment (start 159.2 108.6) (end 159.6 109) (width 0.25) (layer F.Cu) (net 2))
 (segment (start 159.6 109) (end 159.6 111.2) (width 0.25) (layer F.Cu) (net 2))
 (via (at 160.8 112.6) (size 0.8) (drill 0.4) (layers F.Cu B.Cu) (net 2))
 (segment (start 159.6 111.4) (end 160.8 112.6) (width 0.25) (layer F.Cu) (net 2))
 (segment (start 159.6 111.2) (end 159.6 111.4) (width 0.25) (layer F.Cu) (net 2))
 (segment (start 160.8 112.6) (end 161.7 112.6) (width 0.25) (layer B.Cu) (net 2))
 (segment (start 161.7 112.6) (end 161.9 112.4) (width 0.25) (layer B.Cu) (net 2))
 (segment (start 161.9 112.4) (end 161.9 111.2) (width 0.25) (layer B.Cu) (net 2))
 (segment (start 161.9 111.2) (end 162.5 111.2) (width 0.25) (layer B.Cu) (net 2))
 (segment (start 162.5 111.2) (end 162.8 110.9) (width 0.25) (layer B.Cu) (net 2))
 (segment (start 162.8 110.9) (end 163.9 110.9) (width 0.25) (layer B.Cu) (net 2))
 (via (at 156.400988 108.298946) (size 0.8) (drill 0.4) (layers F.Cu B.Cu) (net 2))
 (segment (start 156.400988 107.120988) (end 156.400988 108.298946) (width 0.25) (layer F.Cu) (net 2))
 (segment (start 156.08 106.8) (end 156.400988 107.120988) (width 0.25) (layer F.Cu) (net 2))
 (segment (start 155.3 106.8) (end 156.08 106.8) (width 0.25) (layer F.Cu) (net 2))
 (segment (start 156.400988 108.298946) (end 156.400988 105.600988) (width 0.25) (layer B.Cu) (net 2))
 (segment (start 156.400988 105.600988) (end 155.2 104.4) (width 0.25) (layer B.Cu) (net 2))
 (segment (start 156.601171 106.278829) (end 156.08 106.8) (width 0.25) (layer F.Cu) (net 2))
 (segment (start 156.601171 104.901171) (end 156.601171 106.278829) (width 0.25) (layer F.Cu) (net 2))
 (segment (start 160.55 109.65) (end 162.85 109.65) (width 1) (layer F.Cu) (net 4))
 (segment (start 159.1 107.8) (end 159.9 107.8) (width 0.5) (layer F.Cu) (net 4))
 (segment (start 159.9 107.8) (end 160.5 108.4) (width 0.5) (layer F.Cu) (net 4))
 (segment (start 160.5 108.4) (end 160.5 109.6) (width 0.5) (layer F.Cu) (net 4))
 (segment (start 159.1 107.8) (end 157.5 107.8) (width 0.5) (layer F.Cu) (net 4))
 (via (at 157.5 106.8) (size 0.8) (drill 0.4) (layers F.Cu B.Cu) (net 4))
 (segment (start 157.5 107.75) (end 157.5 106.8) (width 0.5) (layer F.Cu) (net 4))
 (segment (start 157.5 106.8) (end 157.1 106.4) (width 0.5) (layer B.Cu) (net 4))
 (segment (start 157.1 106.4) (end 157.1 104.4) (width 0.5) (layer B.Cu) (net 4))
 (segment (start 157.5 106.8) (end 157.5 109.9) (width 0.5) (layer B.Cu) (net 4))
 (segment (start 157.5 109.9) (end 157.9 110.3) (width 0.5) (layer B.Cu) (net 4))
 (segment (start 157.9 110.3) (end 159.5 110.3) (width 0.5) (layer B.Cu) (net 4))
 (segment (start 162.85 109.65) (end 163.45 109.65) (width 1) (layer F.Cu) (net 4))
 (segment (start 163.45 109.65) (end 163.5 109.6) (width 1) (layer F.Cu) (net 4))
 (segment (start 157.15 104.4) (end 161.3 104.4) (width 0.25) (layer B.Cu) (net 4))
 (segment (start 161.3 104.4) (end 162 103.7) (width 0.25) (layer B.Cu) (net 4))
 (segment (start 162 103.7) (end 163.4 103.7) (width 0.25) (layer B.Cu) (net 4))
 (segment (start 163.4 103.7) (end 163.9 104.2) (width 0.25) (layer B.Cu) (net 4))
 (segment (start 163.9 104.2) (end 163.9 107.5) (width 0.25) (layer B.Cu) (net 4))
 (segment (start 164.95001 108.83682) (end 164.95001 111.64999) (width 0.25) (layer B.Cu) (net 5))
 (segment (start 164.58818 108.47499) (end 164.95001 108.83682) (width 0.25) (layer B.Cu) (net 5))
 (segment (start 163.16249 108.47499) (end 164.58818 108.47499) (width 0.25) (layer B.Cu) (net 5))
 (segment (start 162.4 107.7125) (end 163.16249 108.47499) (width 0.25) (layer B.Cu) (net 5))
 (segment (start 161.7 107.7125) (end 162.4 107.7125) (width 0.25) (layer B.Cu) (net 5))
 (segment (start 164.95001 111.64999) (end 163.9 112.7) (width 0.25) (layer B.Cu) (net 5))
 (via (at 163.9 114.1) (size 0.8) (drill 0.4) (layers F.Cu B.Cu) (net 5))
 (segment (start 163.3 114.7) (end 163.9 114.1) (width 0.25) (layer F.Cu) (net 5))
 (segment (start 160.4 114.7) (end 163.3 114.7) (width 0.25) (layer F.Cu) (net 5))
 (segment (start 163.9 114.1) (end 163.9 112.8) (width 0.25) (layer B.Cu) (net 5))
 (segment (start 159.55 109.035) (end 160.535 109.035) (width 0.25) (layer B.Cu) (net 6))
 (segment (start 160.535 109.035) (end 160.7 109.2) (width 0.25) (layer B.Cu) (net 6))
 (segment (start 160.7 109.2) (end 161.7 109.2) (width 0.25) (layer B.Cu) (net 6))
 (segment (start 161.7 109.2) (end 163.6 109.2) (width 0.25) (layer B.Cu) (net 6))
 (via (at 159.8 112.8) (size 0.8) (drill 0.4) (layers F.Cu B.Cu) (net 6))
 (segment (start 158.9 113.7) (end 159.8 112.8) (width 0.25) (layer F.Cu) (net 6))
 (segment (start 158.9 114.7) (end 158.9 113.7) (width 0.25) (layer F.Cu) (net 6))
 (segment (start 160.84999 110.30001) (end 161.9 109.25) (width 0.25) (layer B.Cu) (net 6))
 (segment (start 160.84999 110.95001) (end 160.84999 110.30001) (width 0.25) (layer B.Cu) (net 6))
 (segment (start 159.8 112) (end 160.84999 110.95001) (width 0.25) (layer B.Cu) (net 6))
 (segment (start 159.8 112.8) (end 159.8 112) (width 0.25) (layer B.Cu) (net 6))
 (segment (start 164.2 106.8) (end 161.8 106.8) (width 1) (layer F.Cu) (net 7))
 (segment (start 161.8 106.8) (end 161.1 106.8) (width 0.25) (layer F.Cu) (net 7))
 (segment (start 152.5 106.8125) (end 153.6875 108) (width 1) (layer F.Cu) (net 9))
 (segment (start 153.6875 108) (end 155.3 108) (width 1) (layer F.Cu) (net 9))
 (segment (start 162.72501 104.62501) (end 162.6 104.5) (width 0.25) (layer B.Cu) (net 10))
 (segment (start 160.58819 105.9) (end 161.2 105.9) (width 0.25) (layer F.Cu) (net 10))
 (segment (start 161.2 105.9) (end 162.6 104.5) (width 0.25) (layer F.Cu) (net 10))
 (via (at 162.6 104.5) (size 0.8) (drill 0.4) (layers F.Cu B.Cu) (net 10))
 (segment (start 159.1 105.9) (end 160.58819 105.9) (width 0.25) (layer F.Cu) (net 10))
 (via (at 154.1 105.6) (size 0.8) (drill 0.4) (layers F.Cu B.Cu) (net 13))
 (segment (start 154.35 105.85) (end 154.1 105.6) (width 0.25) (layer F.Cu) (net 13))
 (segment (start 155.3 105.85) (end 154.35 105.85) (width 0.25) (layer F.Cu) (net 13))
 (segment (start 154.1 105.6) (end 154.1 107.675002) (width 0.25) (layer B.Cu) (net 13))
 (segment (start 154.1 107.675002) (end 154.1 108.7) (width 0.25) (layer B.Cu) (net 13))
 (segment (start 154.1 108.7) (end 153.8 109) (width 0.25) (layer B.Cu) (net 13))
 (segment (start 153.8 109) (end 152.3 109) (width 0.25) (layer B.Cu) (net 13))
 (segment (start 159.05 102.15) (end 159.05 104.05) (width 0.25) (layer F.Cu) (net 3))
 (segment (start 159.05 104.05) (end 159 104) (width 0.25) (layer F.Cu) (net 3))
 (segment (start 159 104) (end 157.5 104) (width 0.25) (layer F.Cu) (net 3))
 (segment (start 157.5 104) (end 157.5 105.8) (width 0.25) (layer F.Cu) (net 3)))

